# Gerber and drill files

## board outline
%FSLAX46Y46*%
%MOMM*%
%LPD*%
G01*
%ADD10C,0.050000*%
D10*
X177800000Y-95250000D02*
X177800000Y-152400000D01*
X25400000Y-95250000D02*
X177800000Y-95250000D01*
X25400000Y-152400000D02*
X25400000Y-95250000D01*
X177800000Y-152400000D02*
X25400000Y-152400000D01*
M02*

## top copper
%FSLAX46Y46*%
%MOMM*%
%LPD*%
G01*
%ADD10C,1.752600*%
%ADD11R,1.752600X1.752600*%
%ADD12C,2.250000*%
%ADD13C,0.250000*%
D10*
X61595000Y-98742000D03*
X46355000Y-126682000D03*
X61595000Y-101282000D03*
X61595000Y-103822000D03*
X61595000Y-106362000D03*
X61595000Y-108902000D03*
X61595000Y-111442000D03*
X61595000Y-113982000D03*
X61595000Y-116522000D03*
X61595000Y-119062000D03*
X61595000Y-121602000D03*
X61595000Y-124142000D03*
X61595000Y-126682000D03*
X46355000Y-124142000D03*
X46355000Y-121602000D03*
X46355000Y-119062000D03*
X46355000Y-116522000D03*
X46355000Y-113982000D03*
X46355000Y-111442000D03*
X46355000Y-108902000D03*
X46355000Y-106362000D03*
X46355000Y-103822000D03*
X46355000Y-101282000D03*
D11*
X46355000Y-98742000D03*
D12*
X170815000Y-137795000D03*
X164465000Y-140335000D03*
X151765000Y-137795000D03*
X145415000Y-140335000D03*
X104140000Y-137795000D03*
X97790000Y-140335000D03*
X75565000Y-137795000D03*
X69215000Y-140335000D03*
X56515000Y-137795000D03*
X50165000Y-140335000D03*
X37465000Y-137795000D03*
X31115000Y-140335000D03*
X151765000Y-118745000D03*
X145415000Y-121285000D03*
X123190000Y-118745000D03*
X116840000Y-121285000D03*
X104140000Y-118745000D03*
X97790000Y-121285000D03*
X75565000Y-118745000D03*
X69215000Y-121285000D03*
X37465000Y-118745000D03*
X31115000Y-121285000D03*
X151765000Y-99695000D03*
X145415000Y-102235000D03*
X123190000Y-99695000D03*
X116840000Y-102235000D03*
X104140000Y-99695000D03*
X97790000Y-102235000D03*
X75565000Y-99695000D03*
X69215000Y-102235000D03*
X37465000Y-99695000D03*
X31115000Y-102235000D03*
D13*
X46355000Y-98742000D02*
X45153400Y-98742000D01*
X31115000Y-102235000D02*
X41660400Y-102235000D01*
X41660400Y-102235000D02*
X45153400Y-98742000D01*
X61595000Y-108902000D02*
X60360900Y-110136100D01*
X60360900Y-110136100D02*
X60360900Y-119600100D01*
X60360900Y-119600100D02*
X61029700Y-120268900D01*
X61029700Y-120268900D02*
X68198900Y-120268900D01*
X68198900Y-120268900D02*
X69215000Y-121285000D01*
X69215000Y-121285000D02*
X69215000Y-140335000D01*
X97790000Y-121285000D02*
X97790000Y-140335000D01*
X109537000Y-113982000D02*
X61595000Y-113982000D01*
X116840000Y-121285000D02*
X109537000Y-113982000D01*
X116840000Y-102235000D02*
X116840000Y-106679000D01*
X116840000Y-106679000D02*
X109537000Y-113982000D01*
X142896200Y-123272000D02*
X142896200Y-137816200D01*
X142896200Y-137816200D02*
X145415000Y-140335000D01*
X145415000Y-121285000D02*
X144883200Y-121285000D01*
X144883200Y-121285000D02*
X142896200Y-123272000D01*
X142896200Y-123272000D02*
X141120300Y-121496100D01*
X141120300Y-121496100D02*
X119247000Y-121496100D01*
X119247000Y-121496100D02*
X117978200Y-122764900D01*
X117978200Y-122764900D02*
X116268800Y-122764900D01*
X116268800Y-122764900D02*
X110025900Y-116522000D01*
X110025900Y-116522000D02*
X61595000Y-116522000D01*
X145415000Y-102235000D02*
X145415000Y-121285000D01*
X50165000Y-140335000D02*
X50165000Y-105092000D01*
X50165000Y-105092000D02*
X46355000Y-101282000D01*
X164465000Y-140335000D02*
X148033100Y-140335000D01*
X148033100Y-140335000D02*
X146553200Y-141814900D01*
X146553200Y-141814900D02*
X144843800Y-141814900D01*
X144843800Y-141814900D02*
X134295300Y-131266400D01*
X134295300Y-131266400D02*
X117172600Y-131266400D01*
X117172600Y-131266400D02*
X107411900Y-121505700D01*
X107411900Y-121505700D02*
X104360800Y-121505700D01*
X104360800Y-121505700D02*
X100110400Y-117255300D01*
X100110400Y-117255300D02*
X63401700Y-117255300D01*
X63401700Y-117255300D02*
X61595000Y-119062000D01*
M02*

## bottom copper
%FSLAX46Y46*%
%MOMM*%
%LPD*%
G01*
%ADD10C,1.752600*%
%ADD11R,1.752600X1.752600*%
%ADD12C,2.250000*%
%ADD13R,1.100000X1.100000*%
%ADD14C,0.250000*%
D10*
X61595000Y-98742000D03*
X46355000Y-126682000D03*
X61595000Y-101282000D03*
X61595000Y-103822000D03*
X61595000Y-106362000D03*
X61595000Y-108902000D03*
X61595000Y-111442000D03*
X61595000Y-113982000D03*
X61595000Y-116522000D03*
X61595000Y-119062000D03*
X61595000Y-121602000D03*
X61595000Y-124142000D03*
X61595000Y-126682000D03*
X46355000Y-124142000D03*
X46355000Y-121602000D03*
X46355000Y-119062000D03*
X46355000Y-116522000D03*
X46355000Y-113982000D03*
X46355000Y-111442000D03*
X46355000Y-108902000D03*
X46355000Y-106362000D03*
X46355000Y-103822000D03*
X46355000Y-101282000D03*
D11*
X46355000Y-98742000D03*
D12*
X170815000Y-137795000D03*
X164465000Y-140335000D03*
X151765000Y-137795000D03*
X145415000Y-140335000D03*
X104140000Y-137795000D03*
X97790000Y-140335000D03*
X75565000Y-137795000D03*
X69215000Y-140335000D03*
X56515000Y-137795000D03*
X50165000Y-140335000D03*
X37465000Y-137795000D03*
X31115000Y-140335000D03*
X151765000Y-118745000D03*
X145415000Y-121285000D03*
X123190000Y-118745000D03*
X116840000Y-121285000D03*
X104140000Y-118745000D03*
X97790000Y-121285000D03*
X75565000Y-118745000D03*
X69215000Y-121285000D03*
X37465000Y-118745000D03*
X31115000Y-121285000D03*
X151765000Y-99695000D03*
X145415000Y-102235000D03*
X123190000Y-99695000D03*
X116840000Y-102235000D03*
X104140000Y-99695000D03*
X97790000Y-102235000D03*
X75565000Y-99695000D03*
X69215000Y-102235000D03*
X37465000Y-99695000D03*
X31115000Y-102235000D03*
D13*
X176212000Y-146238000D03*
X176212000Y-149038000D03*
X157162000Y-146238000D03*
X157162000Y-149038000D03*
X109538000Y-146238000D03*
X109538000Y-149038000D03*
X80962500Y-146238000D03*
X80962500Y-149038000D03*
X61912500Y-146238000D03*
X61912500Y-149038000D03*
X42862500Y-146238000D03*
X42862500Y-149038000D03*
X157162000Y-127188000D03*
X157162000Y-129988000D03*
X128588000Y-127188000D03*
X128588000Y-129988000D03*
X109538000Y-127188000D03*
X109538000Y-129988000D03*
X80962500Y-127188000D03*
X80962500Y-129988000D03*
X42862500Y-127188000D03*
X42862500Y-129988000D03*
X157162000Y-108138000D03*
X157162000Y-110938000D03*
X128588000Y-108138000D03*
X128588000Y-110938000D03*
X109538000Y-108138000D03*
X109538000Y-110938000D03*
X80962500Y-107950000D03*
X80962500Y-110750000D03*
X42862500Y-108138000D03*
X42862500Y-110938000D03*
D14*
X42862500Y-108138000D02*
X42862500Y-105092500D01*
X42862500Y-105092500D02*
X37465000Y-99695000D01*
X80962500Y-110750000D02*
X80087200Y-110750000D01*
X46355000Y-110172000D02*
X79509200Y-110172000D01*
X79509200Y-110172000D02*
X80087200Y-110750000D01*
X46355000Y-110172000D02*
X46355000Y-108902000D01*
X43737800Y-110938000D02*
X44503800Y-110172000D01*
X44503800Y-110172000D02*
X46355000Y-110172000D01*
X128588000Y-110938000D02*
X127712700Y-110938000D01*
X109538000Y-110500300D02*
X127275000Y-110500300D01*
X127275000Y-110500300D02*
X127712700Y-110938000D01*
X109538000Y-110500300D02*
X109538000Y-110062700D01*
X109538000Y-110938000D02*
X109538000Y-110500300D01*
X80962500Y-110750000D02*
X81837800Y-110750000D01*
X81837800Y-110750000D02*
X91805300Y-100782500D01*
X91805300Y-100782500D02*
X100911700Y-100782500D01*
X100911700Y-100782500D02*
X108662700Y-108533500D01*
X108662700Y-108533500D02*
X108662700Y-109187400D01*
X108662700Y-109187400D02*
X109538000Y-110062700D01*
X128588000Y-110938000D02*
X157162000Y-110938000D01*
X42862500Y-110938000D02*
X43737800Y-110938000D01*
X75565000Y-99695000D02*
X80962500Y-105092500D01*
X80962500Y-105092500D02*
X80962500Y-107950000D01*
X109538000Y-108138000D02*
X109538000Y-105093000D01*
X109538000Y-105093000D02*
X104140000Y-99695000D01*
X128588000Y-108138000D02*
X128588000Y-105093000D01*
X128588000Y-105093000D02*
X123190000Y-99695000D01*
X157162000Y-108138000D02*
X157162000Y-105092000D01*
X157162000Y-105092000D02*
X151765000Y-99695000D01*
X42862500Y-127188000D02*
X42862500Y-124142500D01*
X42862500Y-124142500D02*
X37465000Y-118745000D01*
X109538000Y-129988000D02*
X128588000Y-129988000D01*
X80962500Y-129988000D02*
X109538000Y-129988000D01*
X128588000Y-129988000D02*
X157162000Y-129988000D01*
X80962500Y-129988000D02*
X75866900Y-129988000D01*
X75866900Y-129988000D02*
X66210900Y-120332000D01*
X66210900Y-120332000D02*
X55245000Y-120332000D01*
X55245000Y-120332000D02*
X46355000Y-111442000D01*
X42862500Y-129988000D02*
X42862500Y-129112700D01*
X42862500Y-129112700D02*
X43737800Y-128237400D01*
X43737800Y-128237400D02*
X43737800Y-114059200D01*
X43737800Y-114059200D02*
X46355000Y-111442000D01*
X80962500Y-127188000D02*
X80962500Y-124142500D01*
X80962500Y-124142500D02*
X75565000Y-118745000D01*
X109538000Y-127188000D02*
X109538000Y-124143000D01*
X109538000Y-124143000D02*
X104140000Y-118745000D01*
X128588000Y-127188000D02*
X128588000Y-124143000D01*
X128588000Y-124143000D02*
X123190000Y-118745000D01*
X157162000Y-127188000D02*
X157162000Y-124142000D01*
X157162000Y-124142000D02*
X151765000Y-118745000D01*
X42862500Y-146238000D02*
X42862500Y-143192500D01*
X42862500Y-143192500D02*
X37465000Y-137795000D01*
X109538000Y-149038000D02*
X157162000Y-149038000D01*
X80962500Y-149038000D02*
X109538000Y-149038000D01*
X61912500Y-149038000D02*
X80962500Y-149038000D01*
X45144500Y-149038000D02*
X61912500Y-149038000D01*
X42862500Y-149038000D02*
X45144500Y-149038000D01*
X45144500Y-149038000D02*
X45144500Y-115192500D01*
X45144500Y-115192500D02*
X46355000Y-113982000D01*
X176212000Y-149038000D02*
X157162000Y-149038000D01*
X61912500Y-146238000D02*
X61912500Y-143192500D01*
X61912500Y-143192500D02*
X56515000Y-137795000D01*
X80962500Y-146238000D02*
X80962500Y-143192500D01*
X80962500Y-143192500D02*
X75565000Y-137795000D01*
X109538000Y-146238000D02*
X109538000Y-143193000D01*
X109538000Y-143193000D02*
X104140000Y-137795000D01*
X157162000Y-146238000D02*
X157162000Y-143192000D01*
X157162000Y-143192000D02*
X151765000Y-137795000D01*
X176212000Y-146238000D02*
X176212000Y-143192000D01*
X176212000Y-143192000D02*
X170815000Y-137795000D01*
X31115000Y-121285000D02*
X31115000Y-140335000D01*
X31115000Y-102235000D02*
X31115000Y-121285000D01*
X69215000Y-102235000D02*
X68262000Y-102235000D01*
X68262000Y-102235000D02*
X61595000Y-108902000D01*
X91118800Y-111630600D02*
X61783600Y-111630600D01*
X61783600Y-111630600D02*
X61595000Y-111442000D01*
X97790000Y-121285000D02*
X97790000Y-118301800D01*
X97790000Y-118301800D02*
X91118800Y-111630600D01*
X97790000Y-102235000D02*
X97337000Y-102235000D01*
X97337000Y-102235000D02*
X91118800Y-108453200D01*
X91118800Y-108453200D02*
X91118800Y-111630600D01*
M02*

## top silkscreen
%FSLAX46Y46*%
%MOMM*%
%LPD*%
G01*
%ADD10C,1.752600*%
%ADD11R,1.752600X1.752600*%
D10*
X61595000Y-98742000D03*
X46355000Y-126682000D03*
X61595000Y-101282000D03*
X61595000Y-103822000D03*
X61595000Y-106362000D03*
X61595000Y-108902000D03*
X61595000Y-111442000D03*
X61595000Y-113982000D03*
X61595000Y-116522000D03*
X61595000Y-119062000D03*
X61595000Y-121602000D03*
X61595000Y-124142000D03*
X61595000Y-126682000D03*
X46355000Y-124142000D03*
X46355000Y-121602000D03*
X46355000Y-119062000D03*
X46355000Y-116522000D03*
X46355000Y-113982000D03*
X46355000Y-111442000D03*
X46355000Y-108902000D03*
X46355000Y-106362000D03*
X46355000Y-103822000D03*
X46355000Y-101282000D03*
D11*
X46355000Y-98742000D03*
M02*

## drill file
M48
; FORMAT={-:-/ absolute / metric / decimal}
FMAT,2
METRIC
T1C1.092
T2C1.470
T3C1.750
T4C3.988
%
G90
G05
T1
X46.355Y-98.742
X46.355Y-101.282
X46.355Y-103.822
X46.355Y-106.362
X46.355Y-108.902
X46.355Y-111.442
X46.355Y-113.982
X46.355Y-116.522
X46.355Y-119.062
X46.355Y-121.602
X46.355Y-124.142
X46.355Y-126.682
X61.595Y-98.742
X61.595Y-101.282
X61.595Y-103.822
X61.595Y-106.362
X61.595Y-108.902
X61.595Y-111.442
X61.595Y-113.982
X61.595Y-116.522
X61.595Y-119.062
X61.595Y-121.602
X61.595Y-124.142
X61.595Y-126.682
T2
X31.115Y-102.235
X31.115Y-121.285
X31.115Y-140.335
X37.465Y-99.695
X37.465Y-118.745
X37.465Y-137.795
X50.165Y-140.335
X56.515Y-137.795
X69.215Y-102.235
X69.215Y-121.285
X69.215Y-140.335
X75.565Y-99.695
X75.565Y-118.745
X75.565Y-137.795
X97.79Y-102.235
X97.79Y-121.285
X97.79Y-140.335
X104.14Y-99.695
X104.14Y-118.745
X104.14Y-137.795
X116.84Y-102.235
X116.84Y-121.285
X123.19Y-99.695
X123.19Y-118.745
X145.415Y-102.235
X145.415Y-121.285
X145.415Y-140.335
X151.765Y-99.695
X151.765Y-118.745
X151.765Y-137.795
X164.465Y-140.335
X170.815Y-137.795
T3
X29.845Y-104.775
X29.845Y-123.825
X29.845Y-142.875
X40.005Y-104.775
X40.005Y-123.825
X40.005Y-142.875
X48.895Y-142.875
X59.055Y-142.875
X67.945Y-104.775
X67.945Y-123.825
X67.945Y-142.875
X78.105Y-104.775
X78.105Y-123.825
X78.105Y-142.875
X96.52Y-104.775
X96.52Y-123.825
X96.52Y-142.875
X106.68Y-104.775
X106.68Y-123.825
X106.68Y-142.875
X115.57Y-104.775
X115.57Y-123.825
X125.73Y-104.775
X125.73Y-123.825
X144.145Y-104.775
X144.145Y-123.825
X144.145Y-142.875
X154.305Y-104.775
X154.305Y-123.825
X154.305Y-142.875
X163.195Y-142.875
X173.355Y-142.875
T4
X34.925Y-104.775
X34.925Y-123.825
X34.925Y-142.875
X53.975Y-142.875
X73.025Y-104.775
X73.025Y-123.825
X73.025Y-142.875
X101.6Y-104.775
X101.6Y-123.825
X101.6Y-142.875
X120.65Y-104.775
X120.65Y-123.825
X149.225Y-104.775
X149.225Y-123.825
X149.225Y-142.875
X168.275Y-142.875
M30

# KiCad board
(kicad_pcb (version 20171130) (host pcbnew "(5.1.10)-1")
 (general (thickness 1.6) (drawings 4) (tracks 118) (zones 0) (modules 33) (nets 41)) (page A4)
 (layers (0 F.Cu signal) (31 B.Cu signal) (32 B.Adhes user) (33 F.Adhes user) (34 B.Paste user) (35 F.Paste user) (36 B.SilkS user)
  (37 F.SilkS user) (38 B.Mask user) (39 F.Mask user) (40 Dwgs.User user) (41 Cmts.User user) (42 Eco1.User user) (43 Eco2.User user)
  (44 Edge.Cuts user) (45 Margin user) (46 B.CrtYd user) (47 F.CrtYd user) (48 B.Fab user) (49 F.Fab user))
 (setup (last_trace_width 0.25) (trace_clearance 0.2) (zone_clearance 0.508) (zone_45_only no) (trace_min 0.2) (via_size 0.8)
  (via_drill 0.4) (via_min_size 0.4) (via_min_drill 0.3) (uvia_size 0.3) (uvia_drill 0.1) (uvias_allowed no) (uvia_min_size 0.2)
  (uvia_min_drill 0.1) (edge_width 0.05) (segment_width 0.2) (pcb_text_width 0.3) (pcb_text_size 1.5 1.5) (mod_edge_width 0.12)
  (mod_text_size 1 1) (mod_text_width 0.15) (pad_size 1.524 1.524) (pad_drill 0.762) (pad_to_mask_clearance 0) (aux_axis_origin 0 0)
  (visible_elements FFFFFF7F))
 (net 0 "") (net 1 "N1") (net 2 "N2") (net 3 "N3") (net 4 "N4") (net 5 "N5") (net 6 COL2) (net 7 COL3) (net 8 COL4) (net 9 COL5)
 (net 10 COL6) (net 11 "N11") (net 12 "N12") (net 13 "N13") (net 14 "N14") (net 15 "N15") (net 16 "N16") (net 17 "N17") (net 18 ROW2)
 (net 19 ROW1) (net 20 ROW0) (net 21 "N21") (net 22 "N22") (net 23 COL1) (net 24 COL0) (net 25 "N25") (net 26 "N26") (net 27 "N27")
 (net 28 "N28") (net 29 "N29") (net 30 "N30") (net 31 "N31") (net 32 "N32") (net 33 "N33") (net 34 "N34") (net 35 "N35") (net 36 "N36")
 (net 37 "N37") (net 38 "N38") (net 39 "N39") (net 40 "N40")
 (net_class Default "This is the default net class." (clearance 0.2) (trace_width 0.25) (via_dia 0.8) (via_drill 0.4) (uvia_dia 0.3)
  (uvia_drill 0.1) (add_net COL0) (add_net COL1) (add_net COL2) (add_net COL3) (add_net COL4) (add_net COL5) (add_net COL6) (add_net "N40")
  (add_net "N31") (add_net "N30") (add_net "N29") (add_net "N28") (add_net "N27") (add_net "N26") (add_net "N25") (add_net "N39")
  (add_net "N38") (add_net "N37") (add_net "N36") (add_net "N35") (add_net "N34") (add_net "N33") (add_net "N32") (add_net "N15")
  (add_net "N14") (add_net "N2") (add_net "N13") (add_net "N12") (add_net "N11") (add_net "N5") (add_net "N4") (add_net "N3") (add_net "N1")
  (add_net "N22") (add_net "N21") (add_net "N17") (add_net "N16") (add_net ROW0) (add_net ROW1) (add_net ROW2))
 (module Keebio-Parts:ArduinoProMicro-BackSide (layer F.Cu) (at 53.975 112.712 270)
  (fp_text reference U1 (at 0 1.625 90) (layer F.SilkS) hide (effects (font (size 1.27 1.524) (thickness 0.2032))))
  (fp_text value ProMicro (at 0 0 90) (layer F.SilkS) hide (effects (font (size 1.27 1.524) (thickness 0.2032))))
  (pad 24 thru_hole circle (at -13.97 -7.62 270) (size 1.7526 1.7526) (drill 1.0922) (layers *.Cu *.SilkS *.Mask) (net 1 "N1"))
  (pad 12 thru_hole circle (at 13.97 7.62 270) (size 1.7526 1.7526) (drill 1.0922) (layers *.Cu *.SilkS *.Mask) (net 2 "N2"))
  (pad 23 thru_hole circle (at -11.43 -7.62 270) (size 1.7526 1.7526) (drill 1.0922) (layers *.Cu *.SilkS *.Mask) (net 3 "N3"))
  (pad 22 thru_hole circle (at -8.89 -7.62 270) (size 1.7526 1.7526) (drill 1.0922) (layers *.Cu *.SilkS *.Mask) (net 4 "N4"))
  (pad 21 thru_hole circle (at -6.35 -7.62 270) (size 1.7526 1.7526) (drill 1.0922) (layers *.Cu *.SilkS *.Mask) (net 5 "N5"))
  (pad 20 thru_hole circle (at -3.81 -7.62 270) (size 1.7526 1.7526) (drill 1.0922) (layers *.Cu *.SilkS *.Mask) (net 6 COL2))
  (pad 19 thru_hole circle (at -1.27 -7.62 270) (size 1.7526 1.7526) (drill 1.0922) (layers *.Cu *.SilkS *.Mask) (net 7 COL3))
  (pad 18 thru_hole circle (at 1.27 -7.62 270) (size 1.7526 1.7526) (drill 1.0922) (layers *.Cu *.SilkS *.Mask) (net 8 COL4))
  (pad 17 thru_hole circle (at 3.81 -7.62 270) (size 1.7526 1.7526) (drill 1.0922) (layers *.Cu *.SilkS *.Mask) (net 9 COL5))
  (pad 16 thru_hole circle (at 6.35 -7.62 270) (size 1.7526 1.7526) (drill 1.0922) (layers *.Cu *.SilkS *.Mask) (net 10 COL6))
  (pad 15 thru_hole circle (at 8.89 -7.62 270) (size 1.7526 1.7526) (drill 1.0922) (layers *.Cu *.SilkS *.Mask) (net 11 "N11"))
  (pad 14 thru_hole circle (at 11.43 -7.62 270) (size 1.7526 1.7526) (drill 1.0922) (layers *.Cu *.SilkS *.Mask) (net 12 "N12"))
  (pad 13 thru_hole circle (at 13.97 -7.62 270) (size 1.7526 1.7526) (drill 1.0922) (layers *.Cu *.SilkS *.Mask) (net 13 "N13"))
  (pad 11 thru_hole circle (at 11.43 7.62 270) (size 1.7526 1.7526) (drill 1.0922) (layers *.Cu *.SilkS *.Mask) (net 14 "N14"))
  (pad 10 thru_hole circle (at 8.89 7.62 270) (size 1.7526 1.7526) (drill 1.0922) (layers *.Cu *.SilkS *.Mask) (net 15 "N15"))
  (pad 9 thru_hole circle (at 6.35 7.62 270) (size 1.7526 1.7526) (drill 1.0922) (layers *.Cu *.SilkS *.Mask) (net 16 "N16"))
  (pad 8 thru_hole circle (at 3.81 7.62 270) (size 1.7526 1.7526) (drill 1.0922) (layers *.Cu *.SilkS *.Mask) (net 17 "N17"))
  (pad 7 thru_hole circle (at 1.27 7.62 270) (size 1.7526 1.7526) (drill 1.0922) (layers *.Cu *.SilkS *.Mask) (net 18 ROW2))
  (pad 6 thru_hole circle (at -1.27 7.62 270) (size 1.7526 1.7526) (drill 1.0922) (layers *.Cu *.SilkS *.Mask) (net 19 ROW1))
  (pad 5 thru_hole circle (at -3.81 7.62 270) (size 1.7526 1.7526) (drill 1.0922) (layers *.Cu *.SilkS *.Mask) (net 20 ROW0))
  (pad 4 thru_hole circle (at -6.35 7.62 270) (size 1.7526 1.7526) (drill 1.0922) (layers *.Cu *.SilkS *.Mask) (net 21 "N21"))
  (pad 3 thru_hole circle (at -8.89 7.62 270) (size 1.7526 1.7526) (drill 1.0922) (layers *.Cu *.SilkS *.Mask) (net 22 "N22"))
  (pad 2 thru_hole circle (at -11.43 7.62 270) (size 1.7526 1.7526) (drill 1.0922) (layers *.Cu *.SilkS *.Mask) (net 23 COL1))
  (pad 1 thru_hole rect (at -13.97 7.62 270) (size 1.7526 1.7526) (drill 1.0922) (layers *.Cu *.SilkS *.Mask) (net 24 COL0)))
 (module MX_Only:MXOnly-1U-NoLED (layer F.Cu) (at 168.275 142.875)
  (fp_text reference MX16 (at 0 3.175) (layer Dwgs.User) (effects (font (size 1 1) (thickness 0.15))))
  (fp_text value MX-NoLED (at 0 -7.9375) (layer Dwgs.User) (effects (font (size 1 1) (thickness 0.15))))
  (pad 2 thru_hole circle (at 2.54 -5.08) (size 2.25 2.25) (drill 1.47) (layers *.Cu B.Mask) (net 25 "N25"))
  (pad "" np_thru_hole circle (at 0 0) (size 3.9878 3.9878) (drill 3.9878) (layers *.Cu *.Mask))
  (pad 1 thru_hole circle (at -3.81 -2.54) (size 2.25 2.25) (drill 1.47) (layers *.Cu B.Mask) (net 10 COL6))
  (pad "" np_thru_hole circle (at -5.08 0 48.0996) (size 1.75 1.75) (drill 1.75) (layers *.Cu *.Mask))
  (pad "" np_thru_hole circle (at 5.08 0 48.0996) (size 1.75 1.75) (drill 1.75) (layers *.Cu *.Mask)))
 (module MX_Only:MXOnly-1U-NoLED (layer F.Cu) (at 149.225 142.875)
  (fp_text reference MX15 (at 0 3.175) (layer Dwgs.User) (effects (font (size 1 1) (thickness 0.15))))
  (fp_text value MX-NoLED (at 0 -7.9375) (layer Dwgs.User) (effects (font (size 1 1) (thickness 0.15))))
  (pad 2 thru_hole circle (at 2.54 -5.08) (size 2.25 2.25) (drill 1.47) (layers *.Cu B.Mask) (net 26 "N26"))
  (pad "" np_thru_hole circle (at 0 0) (size 3.9878 3.9878) (drill 3.9878) (layers *.Cu *.Mask))
  (pad 1 thru_hole circle (at -3.81 -2.54) (size 2.25 2.25) (drill 1.47) (layers *.Cu B.Mask) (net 9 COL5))
  (pad "" np_thru_hole circle (at -5.08 0 48.0996) (size 1.75 1.75) (drill 1.75) (layers *.Cu *.Mask))
  (pad "" np_thru_hole circle (at 5.08 0 48.0996) (size 1.75 1.75) (drill 1.75) (layers *.Cu *.Mask)))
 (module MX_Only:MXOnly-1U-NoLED (layer F.Cu) (at 101.6 142.875)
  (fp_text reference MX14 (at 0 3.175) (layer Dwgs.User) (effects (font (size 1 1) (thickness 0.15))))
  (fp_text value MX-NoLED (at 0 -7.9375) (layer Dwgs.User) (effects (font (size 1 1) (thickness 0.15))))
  (pad 2 thru_hole circle (at 2.54 -5.08) (size 2.25 2.25) (drill 1.47) (layers *.Cu B.Mask) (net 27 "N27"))
  (pad "" np_thru_hole circle (at 0 0) (size 3.9878 3.9878) (drill 3.9878) (layers *.Cu *.Mask))
  (pad 1 thru_hole circle (at -3.81 -2.54) (size 2.25 2.25) (drill 1.47) (layers *.Cu B.Mask) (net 7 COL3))
  (pad "" np_thru_hole circle (at -5.08 0 48.0996) (size 1.75 1.75) (drill 1.75) (layers *.Cu *.Mask))
  (pad "" np_thru_hole circle (at 5.08 0 48.0996) (size 1.75 1.75) (drill 1.75) (layers *.Cu *.Mask)))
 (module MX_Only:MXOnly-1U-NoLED (layer F.Cu) (at 73.025 142.875)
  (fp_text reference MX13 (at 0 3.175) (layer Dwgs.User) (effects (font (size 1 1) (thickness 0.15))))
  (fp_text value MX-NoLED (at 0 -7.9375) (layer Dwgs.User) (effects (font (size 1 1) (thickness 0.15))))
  (pad 2 thru_hole circle (at 2.54 -5.08) (size 2.25 2.25) (drill 1.47) (layers *.Cu B.Mask) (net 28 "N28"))
  (pad "" np_thru_hole circle (at 0 0) (size 3.9878 3.9878) (drill 3.9878) (layers *.Cu *.Mask))
  (pad 1 thru_hole circle (at -3.81 -2.54) (size 2.25 2.25) (drill 1.47) (layers *.Cu B.Mask) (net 6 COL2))
  (pad "" np_thru_hole circle (at -5.08 0 48.0996) (size 1.75 1.75) (drill 1.75) (layers *.Cu *.Mask))
  (pad "" np_thru_hole circle (at 5.08 0 48.0996) (size 1.75 1.75) (drill 1.75) (layers *.Cu *.Mask)))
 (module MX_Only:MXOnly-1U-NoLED (layer F.Cu) (at 53.975 142.875)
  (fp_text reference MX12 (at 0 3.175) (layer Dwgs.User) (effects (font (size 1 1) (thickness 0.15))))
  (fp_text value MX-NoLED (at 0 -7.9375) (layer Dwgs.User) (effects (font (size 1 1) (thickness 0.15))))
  (pad 2 thru_hole circle (at 2.54 -5.08) (size 2.25 2.25) (drill 1.47) (layers *.Cu B.Mask) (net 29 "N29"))
  (pad "" np_thru_hole circle (at 0 0) (size 3.9878 3.9878) (drill 3.9878) (layers *.Cu *.Mask))
  (pad 1 thru_hole circle (at -3.81 -2.54) (size 2.25 2.25) (drill 1.47) (layers *.Cu B.Mask) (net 23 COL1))
  (pad "" np_thru_hole circle (at -5.08 0 48.0996) (size 1.75 1.75) (drill 1.75) (layers *.Cu *.Mask))
  (pad "" np_thru_hole circle (at 5.08 0 48.0996) (size 1.75 1.75) (drill 1.75) (layers *.Cu *.Mask)))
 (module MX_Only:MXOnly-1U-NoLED (layer F.Cu) (at 34.925 142.875)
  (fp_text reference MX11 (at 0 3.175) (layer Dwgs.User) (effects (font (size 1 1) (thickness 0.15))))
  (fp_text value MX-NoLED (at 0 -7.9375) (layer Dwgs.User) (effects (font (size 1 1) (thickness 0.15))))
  (pad 2 thru_hole circle (at 2.54 -5.08) (size 2.25 2.25) (drill 1.47) (layers *.Cu B.Mask) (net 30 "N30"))
  (pad "" np_thru_hole circle (at 0 0) (size 3.9878 3.9878) (drill 3.9878) (layers *.Cu *.Mask))
  (pad 1 thru_hole circle (at -3.81 -2.54) (size 2.25 2.25) (drill 1.47) (layers *.Cu B.Mask) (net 24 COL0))
  (pad "" np_thru_hole circle (at -5.08 0 48.0996) (size 1.75 1.75) (drill 1.75) (layers *.Cu *.Mask))
  (pad "" np_thru_hole circle (at 5.08 0 48.0996) (size 1.75 1.75) (drill 1.75) (layers *.Cu *.Mask)))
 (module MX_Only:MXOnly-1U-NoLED (layer F.Cu) (at 149.225 123.825)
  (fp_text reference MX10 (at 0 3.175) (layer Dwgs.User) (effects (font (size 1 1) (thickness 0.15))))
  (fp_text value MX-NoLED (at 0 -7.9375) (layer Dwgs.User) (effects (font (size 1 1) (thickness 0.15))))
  (pad 2 thru_hole circle (at 2.54 -5.08) (size 2.25 2.25) (drill 1.47) (layers *.Cu B.Mask) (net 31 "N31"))
  (pad "" np_thru_hole circle (at 0 0) (size 3.9878 3.9878) (drill 3.9878) (layers *.Cu *.Mask))
  (pad 1 thru_hole circle (at -3.81 -2.54) (size 2.25 2.25) (drill 1.47) (layers *.Cu B.Mask) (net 9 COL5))
  (pad "" np_thru_hole circle (at -5.08 0 48.0996) (size 1.75 1.75) (drill 1.75) (layers *.Cu *.Mask))
  (pad "" np_thru_hole circle (at 5.08 0 48.0996) (size 1.75 1.75) (drill 1.75) (layers *.Cu *.Mask)))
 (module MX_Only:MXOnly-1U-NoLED (layer F.Cu) (at 120.65 123.825)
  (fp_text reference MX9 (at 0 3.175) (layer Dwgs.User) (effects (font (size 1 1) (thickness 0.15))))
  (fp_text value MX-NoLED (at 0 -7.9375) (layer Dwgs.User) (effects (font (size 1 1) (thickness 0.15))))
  (pad 2 thru_hole circle (at 2.54 -5.08) (size 2.25 2.25) (drill 1.47) (layers *.Cu B.Mask) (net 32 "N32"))
  (pad "" np_thru_hole circle (at 0 0) (size 3.9878 3.9878) (drill 3.9878) (layers *.Cu *.Mask))
  (pad 1 thru_hole circle (at -3.81 -2.54) (size 2.25 2.25) (drill 1.47) (layers *.Cu B.Mask) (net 8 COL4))
  (pad "" np_thru_hole circle (at -5.08 0 48.0996) (size 1.75 1.75) (drill 1.75) (layers *.Cu *.Mask))
  (pad "" np_thru_hole circle (at 5.08 0 48.0996) (size 1.75 1.75) (drill 1.75) (layers *.Cu *.Mask)))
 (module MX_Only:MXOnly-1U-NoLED (layer F.Cu) (at 101.6 123.825)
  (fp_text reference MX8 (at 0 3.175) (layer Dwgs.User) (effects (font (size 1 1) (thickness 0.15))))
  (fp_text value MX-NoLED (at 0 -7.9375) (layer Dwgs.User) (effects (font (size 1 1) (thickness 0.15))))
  (pad 2 thru_hole circle (at 2.54 -5.08) (size 2.25 2.25) (drill 1.47) (layers *.Cu B.Mask) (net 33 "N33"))
  (pad "" np_thru_hole circle (at 0 0) (size 3.9878 3.9878) (drill 3.9878) (layers *.Cu *.Mask))
  (pad 1 thru_hole circle (at -3.81 -2.54) (size 2.25 2.25) (drill 1.47) (layers *.Cu B.Mask) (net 7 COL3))
  (pad "" np_thru_hole circle (at -5.08 0 48.0996) (size 1.75 1.75) (drill 1.75) (layers *.Cu *.Mask))
  (pad "" np_thru_hole circle (at 5.08 0 48.0996) (size 1.75 1.75) (drill 1.75) (layers *.Cu *.Mask)))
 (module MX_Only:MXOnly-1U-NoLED (layer F.Cu) (at 73.025 123.825)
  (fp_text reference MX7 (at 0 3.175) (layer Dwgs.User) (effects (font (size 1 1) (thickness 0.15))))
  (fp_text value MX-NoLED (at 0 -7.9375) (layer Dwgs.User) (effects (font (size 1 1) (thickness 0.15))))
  (pad 2 thru_hole circle (at 2.54 -5.08) (size 2.25 2.25) (drill 1.47) (layers *.Cu B.Mask) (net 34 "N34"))
  (pad "" np_thru_hole circle (at 0 0) (size 3.9878 3.9878) (drill 3.9878) (layers *.Cu *.Mask))
  (pad 1 thru_hole circle (at -3.81 -2.54) (size 2.25 2.25) (drill 1.47) (layers *.Cu B.Mask) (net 6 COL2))
  (pad "" np_thru_hole circle (at -5.08 0 48.0996) (size 1.75 1.75) (drill 1.75) (layers *.Cu *.Mask))
  (pad "" np_thru_hole circle (at 5.08 0 48.0996) (size 1.75 1.75) (drill 1.75) (layers *.Cu *.Mask)))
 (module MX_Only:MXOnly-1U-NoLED (layer F.Cu) (at 34.925 123.825)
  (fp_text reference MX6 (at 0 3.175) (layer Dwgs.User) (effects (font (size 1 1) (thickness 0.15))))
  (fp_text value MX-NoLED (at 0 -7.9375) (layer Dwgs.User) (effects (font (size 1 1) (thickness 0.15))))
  (pad 2 thru_hole circle (at 2.54 -5.08) (size 2.25 2.25) (drill 1.47) (layers *.Cu B.Mask) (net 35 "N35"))
  (pad "" np_thru_hole circle (at 0 0) (size 3.9878 3.9878) (drill 3.9878) (layers *.Cu *.Mask))
  (pad 1 thru_hole circle (at -3.81 -2.54) (size 2.25 2.25) (drill 1.47) (layers *.Cu B.Mask) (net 24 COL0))
  (pad "" np_thru_hole circle (at -5.08 0 48.0996) (size 1.75 1.75) (drill 1.75) (layers *.Cu *.Mask))
  (pad "" np_thru_hole circle (at 5.08 0 48.0996) (size 1.75 1.75) (drill 1.75) (layers *.Cu *.Mask)))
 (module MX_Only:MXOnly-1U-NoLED (layer F.Cu) (at 149.225 104.775)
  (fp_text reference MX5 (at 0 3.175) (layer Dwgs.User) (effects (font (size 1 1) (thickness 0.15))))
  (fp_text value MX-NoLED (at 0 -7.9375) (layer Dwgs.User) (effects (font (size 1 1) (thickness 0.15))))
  (pad 2 thru_hole circle (at 2.54 -5.08) (size 2.25 2.25) (drill 1.47) (layers *.Cu B.Mask) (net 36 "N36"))
  (pad "" np_thru_hole circle (at 0 0) (size 3.9878 3.9878) (drill 3.9878) (layers *.Cu *.Mask))
  (pad 1 thru_hole circle (at -3.81 -2.54) (size 2.25 2.25) (drill 1.47) (layers *.Cu B.Mask) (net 9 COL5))
  (pad "" np_thru_hole circle (at -5.08 0 48.0996) (size 1.75 1.75) (drill 1.75) (layers *.Cu *.Mask))
  (pad "" np_thru_hole circle (at 5.08 0 48.0996) (size 1.75 1.75) (drill 1.75) (layers *.Cu *.Mask)))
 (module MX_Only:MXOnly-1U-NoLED (layer F.Cu) (at 120.65 104.775)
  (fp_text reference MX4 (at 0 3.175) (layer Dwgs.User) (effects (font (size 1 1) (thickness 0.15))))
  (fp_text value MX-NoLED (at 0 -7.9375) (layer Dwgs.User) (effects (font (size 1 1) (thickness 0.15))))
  (pad 2 thru_hole circle (at 2.54 -5.08) (size 2.25 2.25) (drill 1.47) (layers *.Cu B.Mask) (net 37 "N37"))
  (pad "" np_thru_hole circle (at 0 0) (size 3.9878 3.9878) (drill 3.9878) (layers *.Cu *.Mask))
  (pad 1 thru_hole circle (at -3.81 -2.54) (size 2.25 2.25) (drill 1.47) (layers *.Cu B.Mask) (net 8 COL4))
  (pad "" np_thru_hole circle (at -5.08 0 48.0996) (size 1.75 1.75) (drill 1.75) (layers *.Cu *.Mask))
  (pad "" np_thru_hole circle (at 5.08 0 48.0996) (size 1.75 1.75) (drill 1.75) (layers *.Cu *.Mask)))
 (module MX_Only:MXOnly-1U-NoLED (layer F.Cu) (at 101.6 104.775)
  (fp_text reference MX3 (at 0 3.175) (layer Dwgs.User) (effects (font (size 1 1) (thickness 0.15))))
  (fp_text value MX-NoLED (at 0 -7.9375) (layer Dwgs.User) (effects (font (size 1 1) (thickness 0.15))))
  (pad 2 thru_hole circle (at 2.54 -5.08) (size 2.25 2.25) (drill 1.47) (layers *.Cu B.Mask) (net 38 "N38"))
  (pad "" np_thru_hole circle (at 0 0) (size 3.9878 3.9878) (drill 3.9878) (layers *.Cu *.Mask))
  (pad 1 thru_hole circle (at -3.81 -2.54) (size 2.25 2.25) (drill 1.47) (layers *.Cu B.Mask) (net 7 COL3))
  (pad "" np_thru_hole circle (at -5.08 0 48.0996) (size 1.75 1.75) (drill 1.75) (layers *.Cu *.Mask))
  (pad "" np_thru_hole circle (at 5.08 0 48.0996) (size 1.75 1.75) (drill 1.75) (layers *.Cu *.Mask)))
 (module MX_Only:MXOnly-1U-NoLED (layer F.Cu) (at 73.025 104.775)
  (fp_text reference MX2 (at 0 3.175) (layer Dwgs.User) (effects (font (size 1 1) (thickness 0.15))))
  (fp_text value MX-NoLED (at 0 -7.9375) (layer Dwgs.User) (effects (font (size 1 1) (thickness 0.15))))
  (pad 2 thru_hole circle (at 2.54 -5.08) (size 2.25 2.25) (drill 1.47) (layers *.Cu B.Mask) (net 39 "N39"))
  (pad "" np_thru_hole circle (at 0 0) (size 3.9878 3.9878) (drill 3.9878) (layers *.Cu *.Mask))
  (pad 1 thru_hole circle (at -3.81 -2.54) (size 2.25 2.25) (drill 1.47) (layers *.Cu B.Mask) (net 6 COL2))
  (pad "" np_thru_hole circle (at -5.08 0 48.0996) (size 1.75 1.75) (drill 1.75) (layers *.Cu *.Mask))
  (pad "" np_thru_hole circle (at 5.08 0 48.0996) (size 1.75 1.75) (drill 1.75) (layers *.Cu *.Mask)))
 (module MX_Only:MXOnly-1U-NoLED (layer F.Cu) (at 34.925 104.775)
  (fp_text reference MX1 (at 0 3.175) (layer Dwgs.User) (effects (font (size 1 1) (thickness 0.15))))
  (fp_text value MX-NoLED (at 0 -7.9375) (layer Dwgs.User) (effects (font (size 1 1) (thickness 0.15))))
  (pad 2 thru_hole circle (at 2.54 -5.08) (size 2.25 2.25) (drill 1.47) (layers *.Cu B.Mask) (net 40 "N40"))
  (pad "" np_thru_hole circle (at 0 0) (size 3.9878 3.9878) (drill 3.9878) (layers *.Cu *.Mask))
  (pad 1 thru_hole circle (at -3.81 -2.54) (size 2.25 2.25) (drill 1.47) (layers *.Cu B.Mask) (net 24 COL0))
  (pad "" np_thru_hole circle (at -5.08 0 48.0996) (size 1.75 1.75) (drill 1.75) (layers *.Cu *.Mask))
  (pad "" np_thru_hole circle (at 5.08 0 48.0996) (size 1.75 1.75) (drill 1.75) (layers *.Cu *.Mask)))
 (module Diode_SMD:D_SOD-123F (layer B.Cu) (at 176.212 147.638 90)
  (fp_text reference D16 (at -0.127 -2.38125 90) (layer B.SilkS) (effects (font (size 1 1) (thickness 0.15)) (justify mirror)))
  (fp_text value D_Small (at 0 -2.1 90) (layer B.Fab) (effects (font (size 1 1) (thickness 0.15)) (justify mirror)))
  (pad 2 smd rect (at 1.4 0 90) (size 1.1 1.1) (layers B.Cu B.Paste B.Mask) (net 25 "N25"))
  (pad 1 smd rect (at -1.4 0 90) (size 1.1 1.1) (layers B.Cu B.Paste B.Mask) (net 18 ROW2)))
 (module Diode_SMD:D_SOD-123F (layer B.Cu) (at 157.162 147.638 90)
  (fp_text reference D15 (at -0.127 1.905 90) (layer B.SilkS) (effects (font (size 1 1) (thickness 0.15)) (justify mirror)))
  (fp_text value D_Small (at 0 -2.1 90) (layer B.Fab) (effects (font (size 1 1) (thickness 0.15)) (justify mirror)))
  (pad 2 smd rect (at 1.4 0 90) (size 1.1 1.1) (layers B.Cu B.Paste B.Mask) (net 26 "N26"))
  (pad 1 smd rect (at -1.4 0 90) (size 1.1 1.1) (layers B.Cu B.Paste B.Mask) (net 18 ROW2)))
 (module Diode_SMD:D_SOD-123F (layer B.Cu) (at 109.538 147.638 90)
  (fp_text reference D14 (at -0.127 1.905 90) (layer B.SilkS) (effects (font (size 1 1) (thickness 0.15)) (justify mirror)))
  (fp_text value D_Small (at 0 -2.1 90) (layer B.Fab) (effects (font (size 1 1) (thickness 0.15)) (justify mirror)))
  (pad 2 smd rect (at 1.4 0 90) (size 1.1 1.1) (layers B.Cu B.Paste B.Mask) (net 27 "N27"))
  (pad 1 smd rect (at -1.4 0 90) (size 1.1 1.1) (layers B.Cu B.Paste B.Mask) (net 18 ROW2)))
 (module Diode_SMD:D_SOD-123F (layer B.Cu) (at 80.9625 147.638 90)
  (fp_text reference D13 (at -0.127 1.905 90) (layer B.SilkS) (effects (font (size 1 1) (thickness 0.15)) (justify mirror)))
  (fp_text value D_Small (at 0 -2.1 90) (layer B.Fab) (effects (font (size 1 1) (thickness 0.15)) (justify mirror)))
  (pad 2 smd rect (at 1.4 0 90) (size 1.1 1.1) (layers B.Cu B.Paste B.Mask) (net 28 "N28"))
  (pad 1 smd rect (at -1.4 0 90) (size 1.1 1.1) (layers B.Cu B.Paste B.Mask) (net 18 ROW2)))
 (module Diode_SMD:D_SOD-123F (layer B.Cu) (at 61.9125 147.638 90)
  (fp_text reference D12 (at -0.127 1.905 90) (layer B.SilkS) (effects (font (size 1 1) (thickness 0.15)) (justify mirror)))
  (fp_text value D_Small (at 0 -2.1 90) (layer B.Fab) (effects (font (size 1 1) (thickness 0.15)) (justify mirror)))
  (pad 2 smd rect (at 1.4 0 90) (size 1.1 1.1) (layers B.Cu B.Paste B.Mask) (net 29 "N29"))
  (pad 1 smd rect (at -1.4 0 90) (size 1.1 1.1) (layers B.Cu B.Paste B.Mask) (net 18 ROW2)))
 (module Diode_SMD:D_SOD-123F (layer B.Cu) (at 42.8625 147.638 90)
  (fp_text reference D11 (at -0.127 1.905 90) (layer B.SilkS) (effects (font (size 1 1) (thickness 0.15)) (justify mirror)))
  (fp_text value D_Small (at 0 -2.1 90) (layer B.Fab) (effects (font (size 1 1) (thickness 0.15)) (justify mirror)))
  (pad 2 smd rect (at 1.4 0 90) (size 1.1 1.1) (layers B.Cu B.Paste B.Mask) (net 30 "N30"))
  (pad 1 smd rect (at -1.4 0 90) (size 1.1 1.1) (layers B.Cu B.Paste B.Mask) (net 18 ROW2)))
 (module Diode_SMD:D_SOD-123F (layer B.Cu) (at 157.162 128.588 90)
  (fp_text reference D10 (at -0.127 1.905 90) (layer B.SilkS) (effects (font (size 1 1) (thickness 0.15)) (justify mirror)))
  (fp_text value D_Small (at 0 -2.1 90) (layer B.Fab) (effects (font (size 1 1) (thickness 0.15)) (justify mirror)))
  (pad 2 smd rect (at 1.4 0 90) (size 1.1 1.1) (layers B.Cu B.Paste B.Mask) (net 31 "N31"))
  (pad 1 smd rect (at -1.4 0 90) (size 1.1 1.1) (layers B.Cu B.Paste B.Mask) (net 19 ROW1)))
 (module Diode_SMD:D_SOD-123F (layer B.Cu) (at 128.588 128.588 90)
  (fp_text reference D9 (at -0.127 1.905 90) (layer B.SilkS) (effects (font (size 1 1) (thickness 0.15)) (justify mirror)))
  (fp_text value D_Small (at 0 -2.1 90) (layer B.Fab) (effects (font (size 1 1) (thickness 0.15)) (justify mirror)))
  (pad 2 smd rect (at 1.4 0 90) (size 1.1 1.1) (layers B.Cu B.Paste B.Mask) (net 32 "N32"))
  (pad 1 smd rect (at -1.4 0 90) (size 1.1 1.1) (layers B.Cu B.Paste B.Mask) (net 19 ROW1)))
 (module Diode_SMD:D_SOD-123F (layer B.Cu) (at 109.538 128.588 90)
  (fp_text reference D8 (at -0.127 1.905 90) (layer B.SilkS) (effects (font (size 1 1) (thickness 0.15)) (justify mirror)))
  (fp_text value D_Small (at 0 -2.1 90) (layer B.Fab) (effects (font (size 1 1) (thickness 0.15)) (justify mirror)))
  (pad 2 smd rect (at 1.4 0 90) (size 1.1 1.1) (layers B.Cu B.Paste B.Mask) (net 33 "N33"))
  (pad 1 smd rect (at -1.4 0 90) (size 1.1 1.1) (layers B.Cu B.Paste B.Mask) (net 19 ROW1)))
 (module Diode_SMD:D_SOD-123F (layer B.Cu) (at 80.9625 128.588 90)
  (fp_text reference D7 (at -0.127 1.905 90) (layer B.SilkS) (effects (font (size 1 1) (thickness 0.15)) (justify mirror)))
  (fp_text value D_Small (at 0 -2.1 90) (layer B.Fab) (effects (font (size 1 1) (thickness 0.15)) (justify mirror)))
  (pad 2 smd rect (at 1.4 0 90) (size 1.1 1.1) (layers B.Cu B.Paste B.Mask) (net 34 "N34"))
  (pad 1 smd rect (at -1.4 0 90) (size 1.1 1.1) (layers B.Cu B.Paste B.Mask) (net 19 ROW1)))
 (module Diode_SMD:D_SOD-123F (layer B.Cu) (at 42.8625 128.588 90)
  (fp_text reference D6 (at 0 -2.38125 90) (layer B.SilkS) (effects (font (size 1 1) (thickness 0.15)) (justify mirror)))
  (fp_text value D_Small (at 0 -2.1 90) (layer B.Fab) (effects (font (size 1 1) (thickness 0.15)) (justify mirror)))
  (pad 2 smd rect (at 1.4 0 90) (size 1.1 1.1) (layers B.Cu B.Paste B.Mask) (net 35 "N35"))
  (pad 1 smd rect (at -1.4 0 90) (size 1.1 1.1) (layers B.Cu B.Paste B.Mask) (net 19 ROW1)))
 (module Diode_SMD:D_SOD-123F (layer B.Cu) (at 157.162 109.538 90)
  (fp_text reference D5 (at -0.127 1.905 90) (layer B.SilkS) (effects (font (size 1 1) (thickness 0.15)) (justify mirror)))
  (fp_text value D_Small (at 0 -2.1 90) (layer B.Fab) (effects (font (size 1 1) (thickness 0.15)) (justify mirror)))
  (pad 2 smd rect (at 1.4 0 90) (size 1.1 1.1) (layers B.Cu B.Paste B.Mask) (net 36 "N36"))
  (pad 1 smd rect (at -1.4 0 90) (size 1.1 1.1) (layers B.Cu B.Paste B.Mask) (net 20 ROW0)))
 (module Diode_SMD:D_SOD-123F (layer B.Cu) (at 128.588 109.538 90)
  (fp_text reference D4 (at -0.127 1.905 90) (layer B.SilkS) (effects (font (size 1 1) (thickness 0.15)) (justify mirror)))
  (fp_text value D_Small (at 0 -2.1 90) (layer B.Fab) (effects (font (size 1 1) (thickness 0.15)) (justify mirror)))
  (pad 2 smd rect (at 1.4 0 90) (size 1.1 1.1) (layers B.Cu B.Paste B.Mask) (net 37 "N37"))
  (pad 1 smd rect (at -1.4 0 90) (size 1.1 1.1) (layers B.Cu B.Paste B.Mask) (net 20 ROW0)))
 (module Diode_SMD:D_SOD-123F (layer B.Cu) (at 109.538 109.538 90)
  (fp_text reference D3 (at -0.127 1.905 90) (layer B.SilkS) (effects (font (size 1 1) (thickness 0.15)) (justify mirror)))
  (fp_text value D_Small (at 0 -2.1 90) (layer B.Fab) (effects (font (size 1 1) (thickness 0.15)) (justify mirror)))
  (pad 2 smd rect (at 1.4 0 90) (size 1.1 1.1) (layers B.Cu B.Paste B.Mask) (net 38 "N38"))
  (pad 1 smd rect (at -1.4 0 90) (size 1.1 1.1) (layers B.Cu B.Paste B.Mask) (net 20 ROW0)))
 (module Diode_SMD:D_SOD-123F (layer B.Cu) (at 80.9625 109.35 90)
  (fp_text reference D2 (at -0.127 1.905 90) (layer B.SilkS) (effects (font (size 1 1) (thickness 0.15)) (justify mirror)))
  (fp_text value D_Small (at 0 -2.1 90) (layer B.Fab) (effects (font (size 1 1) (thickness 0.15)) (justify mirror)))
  (pad 2 smd rect (at 1.4 0 90) (size 1.1 1.1) (layers B.Cu B.Paste B.Mask) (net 39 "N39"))
  (pad 1 smd rect (at -1.4 0 90) (size 1.1 1.1) (layers B.Cu B.Paste B.Mask) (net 20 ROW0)))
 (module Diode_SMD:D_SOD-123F (layer B.Cu) (at 42.8625 109.538 90)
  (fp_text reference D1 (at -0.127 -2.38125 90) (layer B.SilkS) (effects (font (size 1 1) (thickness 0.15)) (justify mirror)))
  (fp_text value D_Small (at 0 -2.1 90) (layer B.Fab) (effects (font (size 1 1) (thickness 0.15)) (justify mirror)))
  (pad 2 smd rect (at 1.4 0 90) (size 1.1 1.1) (layers B.Cu B.Paste B.Mask) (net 40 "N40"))
  (pad 1 smd rect (at -1.4 0 90) (size 1.1 1.1) (layers B.Cu B.Paste B.Mask) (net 20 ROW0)))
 (gr_line (start 177.8 95.25) (end 177.8 152.4) (layer Edge.Cuts) (width 0.05))
 (gr_line (start 25.4 95.25) (end 177.8 95.25) (layer Edge.Cuts) (width 0.05))
 (gr_line (start 25.4 152.4) (end 25.4 95.25) (layer Edge.Cuts) (width 0.05))
 (gr_line (start 177.8 152.4) (end 25.4 152.4) (layer Edge.Cuts) (width 0.05))
 (segment (start 42.8625 108.138) (end 42.8625 105.0925) (width 0.25) (layer B.Cu) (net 40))
 (segment (start 42.8625 105.0925) (end 37.465 99.695) (width 0.25) (layer B.Cu) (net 40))
 (segment (start 80.9625 110.75) (end 80.0872 110.75) (width 0.25) (layer B.Cu) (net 20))
 (segment (start 46.355 110.172) (end 79.5092 110.172) (width 0.25) (layer B.Cu) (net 20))
 (segment (start 79.5092 110.172) (end 80.0872 110.75) (width 0.25) (layer B.Cu) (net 20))
 (segment (start 46.355 110.172) (end 46.355 108.902) (width 0.25) (layer B.Cu) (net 20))
 (segment (start 43.7378 110.938) (end 44.5038 110.172) (width 0.25) (layer B.Cu) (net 20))
 (segment (start 44.5038 110.172) (end 46.355 110.172) (width 0.25) (layer B.Cu) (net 20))
 (segment (start 128.588 110.938) (end 127.7127 110.938) (width 0.25) (layer B.Cu) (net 20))
 (segment (start 109.538 110.5003) (end 127.275 110.5003) (width 0.25) (layer B.Cu) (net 20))
 (segment (start 127.275 110.5003) (end 127.7127 110.938) (width 0.25) (layer B.Cu) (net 20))
 (segment (start 109.538 110.5003) (end 109.538 110.0627) (width 0.25) (layer B.Cu) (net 20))
 (segment (start 109.538 110.938) (end 109.538 110.5003) (width 0.25) (layer B.Cu) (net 20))
 (segment (start 80.9625 110.75) (end 81.8378 110.75) (width 0.25) (layer B.Cu) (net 20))
 (segment (start 81.8378 110.75) (end 91.8053 100.7825) (width 0.25) (layer B.Cu) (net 20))
 (segment (start 91.8053 100.7825) (end 100.9117 100.7825) (width 0.25) (layer B.Cu) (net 20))
 (segment (start 100.9117 100.7825) (end 108.6627 108.5335) (width 0.25) (layer B.Cu) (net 20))
 (segment (start 108.6627 108.5335) (end 108.6627 109.1874) (width 0.25) (layer B.Cu) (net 20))
 (segment (start 108.6627 109.1874) (end 109.538 110.0627) (width 0.25) (layer B.Cu) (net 20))
 (segment (start 128.588 110.938) (end 157.162 110.938) (width 0.25) (layer B.Cu) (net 20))
 (segment (start 42.8625 110.938) (end 43.7378 110.938) (width 0.25) (layer B.Cu) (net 20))
 (segment (start 75.565 99.695) (end 80.9625 105.0925) (width 0.25) (layer B.Cu) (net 39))
 (segment (start 80.9625 105.0925) (end 80.9625 107.95) (width 0.25) (layer B.Cu) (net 39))
 (segment (start 109.538 108.138) (end 109.538 105.093) (width 0.25) (layer B.Cu) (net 38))
 (segment (start 109.538 105.093) (end 104.14 99.695) (width 0.25) (layer B.Cu) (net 38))
 (segment (start 128.588 108.138) (end 128.588 105.093) (width 0.25) (layer B.Cu) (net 37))
 (segment (start 128.588 105.093) (end 123.19 99.695) (width 0.25) (layer B.Cu) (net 37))
 (segment (start 157.162 108.138) (end 157.162 105.092) (width 0.25) (layer B.Cu) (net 36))
 (segment (start 157.162 105.092) (end 151.765 99.695) (width 0.25) (layer B.Cu) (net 36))
 (segment (start 42.8625 127.188) (end 42.8625 124.1425) (width 0.25) (layer B.Cu) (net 35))
 (segment (start 42.8625 124.1425) (end 37.465 118.745) (width 0.25) (layer B.Cu) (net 35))
 (segment (start 109.538 129.988) (end 128.588 129.988) (width 0.25) (layer B.Cu) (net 19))
 (segment (start 80.9625 129.988) (end 109.538 129.988) (width 0.25) (layer B.Cu) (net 19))
 (segment (start 128.588 129.988) (end 157.162 129.988) (width 0.25) (layer B.Cu) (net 19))
 (segment (start 80.9625 129.988) (end 75.8669 129.988) (width 0.25) (layer B.Cu) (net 19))
 (segment (start 75.8669 129.988) (end 66.2109 120.332) (width 0.25) (layer B.Cu) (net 19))
 (segment (start 66.2109 120.332) (end 55.245 120.332) (width 0.25) (layer B.Cu) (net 19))
 (segment (start 55.245 120.332) (end 46.355 111.442) (width 0.25) (layer B.Cu) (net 19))
 (segment (start 42.8625 129.988) (end 42.8625 129.1127) (width 0.25) (layer B.Cu) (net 19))
 (segment (start 42.8625 129.1127) (end 43.7378 128.2374) (width 0.25) (layer B.Cu) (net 19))
 (segment (start 43.7378 128.2374) (end 43.7378 114.0592) (width 0.25) (layer B.Cu) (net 19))
 (segment (start 43.7378 114.0592) (end 46.355 111.442) (width 0.25) (layer B.Cu) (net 19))
 (segment (start 80.9625 127.188) (end 80.9625 124.1425) (width 0.25) (layer B.Cu) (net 34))
 (segment (start 80.9625 124.1425) (end 75.565 118.745) (width 0.25) (layer B.Cu) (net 34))
 (segment (start 109.538 127.188) (end 109.538 124.143) (width 0.25) (layer B.Cu) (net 33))
 (segment (start 109.538 124.143) (end 104.14 118.745) (width 0.25) (layer B.Cu) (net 33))
 (segment (start 128.588 127.188) (end 128.588 124.143) (width 0.25) (layer B.Cu) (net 32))
 (segment (start 128.588 124.143) (end 123.19 118.745) (width 0.25) (layer B.Cu) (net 32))
 (segment (start 157.162 127.188) (end 157.162 124.142) (width 0.25) (layer B.Cu) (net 31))
 (segment (start 157.162 124.142) (end 151.765 118.745) (width 0.25) (layer B.Cu) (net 31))
 (segment (start 42.8625 146.238) (end 42.8625 143.1925) (width 0.25) (layer B.Cu) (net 30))
 (segment (start 42.8625 143.1925) (end 37.465 137.795) (width 0.25) (layer B.Cu) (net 30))
 (segment (start 109.538 149.038) (end 157.162 149.038) (width 0.25) (layer B.Cu) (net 18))
 (segment (start 80.9625 149.038) (end 109.538 149.038) (width 0.25) (layer B.Cu) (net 18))
 (segment (start 61.9125 149.038) (end 80.9625 149.038) (width 0.25) (layer B.Cu) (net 18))
 (segment (start 45.1445 149.038) (end 61.9125 149.038) (width 0.25) (layer B.Cu) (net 18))
 (segment (start 42.8625 149.038) (end 45.1445 149.038) (width 0.25) (layer B.Cu) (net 18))
 (segment (start 45.1445 149.038) (end 45.1445 115.1925) (width 0.25) (layer B.Cu) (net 18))
 (segment (start 45.1445 115.1925) (end 46.355 113.982) (width 0.25) (layer B.Cu) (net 18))
 (segment (start 176.212 149.038) (end 157.162 149.038) (width 0.25) (layer B.Cu) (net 18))
 (segment (start 61.9125 146.238) (end 61.9125 143.1925) (width 0.25) (layer B.Cu) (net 29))
 (segment (start 61.9125 143.1925) (end 56.515 137.795) (width 0.25) (layer B.Cu) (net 29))
 (segment (start 80.9625 146.238) (end 80.9625 143.1925) (width 0.25) (layer B.Cu) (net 28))
 (segment (start 80.9625 143.1925) (end 75.565 137.795) (width 0.25) (layer B.Cu) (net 28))
 (segment (start 109.538 146.238) (end 109.538 143.193) (width 0.25) (layer B.Cu) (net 27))
 (segment (start 109.538 143.193) (end 104.14 137.795) (width 0.25) (layer B.Cu) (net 27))
 (segment (start 157.162 146.238) (end 157.162 143.192) (width 0.25) (layer B.Cu) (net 26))
 (segment (start 157.162 143.192) (end 151.765 137.795) (width 0.25) (layer B.Cu) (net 26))
 (segment (start 176.212 146.238) (end 176.212 143.192) (width 0.25) (layer B.Cu) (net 25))
 (segment (start 176.212 143.192) (end 170.815 137.795) (width 0.25) (layer B.Cu) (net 25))
 (segment (start 46.355 98.742) (end 45.1534 98.742) (width 0.25) (layer F.Cu) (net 24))
 (segment (start 31.115 102.235) (end 41.6604 102.235) (width 0.25) (layer F.Cu) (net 24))
 (segment (start 41.6604 102.235) (end 45.1534 98.742) (width 0.25) (layer F.Cu) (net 24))
 (segment (start 31.115 121.285) (end 31.115 140.335) (width 0.25) (layer B.Cu) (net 24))
 (segment (start 31.115 102.235) (end 31.115 121.285) (width 0.25) (layer B.Cu) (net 24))
 (segment (start 61.595 108.902) (end 60.3609 110.1361) (width 0.25) (layer F.Cu) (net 6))
 (segment (start 60.3609 110.1361) (end 60.3609 119.6001) (width 0.25) (layer F.Cu) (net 6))
 (segment (start 60.3609 119.6001) (end 61.0297 120.2689) (width 0.25) (layer F.Cu) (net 6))
 (segment (start 61.0297 120.2689) (end 68.1989 120.2689) (width 0.25) (layer F.Cu) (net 6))
 (segment (start 68.1989 120.2689) (end 69.215 121.285) (width 0.25) (layer F.Cu) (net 6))
 (segment (start 69.215 121.285) (end 69.215 140.335) (width 0.25) (layer F.Cu) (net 6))
 (segment (start 69.215 102.235) (end 68.262 102.235) (width 0.25) (layer B.Cu) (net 6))
 (segment (start 68.262 102.235) (end 61.595 108.902) (width 0.25) (layer B.Cu) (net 6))
 (segment (start 91.1188 111.6306) (end 61.7836 111.6306) (width 0.25) (layer B.Cu) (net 7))
 (segment (start 61.7836 111.6306) (end 61.595 111.442) (width 0.25) (layer B.Cu) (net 7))
 (segment (start 97.79 121.285) (end 97.79 118.3018) (width 0.25) (layer B.Cu) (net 7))
 (segment (start 97.79 118.3018) (end 91.1188 111.6306) (width 0.25) (layer B.Cu) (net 7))
 (segment (start 97.79 102.235) (end 97.337 102.235) (width 0.25) (layer B.Cu) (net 7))
 (segment (start 97.337 102.235) (end 91.1188 108.4532) (width 0.25) (layer B.Cu) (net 7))
 (segment (start 91.1188 108.4532) (end 91.1188 111.6306) (width 0.25) (layer B.Cu) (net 7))
 (segment (start 97.79 121.285) (end 97.79 140.335) (width 0.25) (layer F.Cu) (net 7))
 (segment (start 109.537 113.982) (end 61.595 113.982) (width 0.25) (layer F.Cu) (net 8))
 (segment (start 116.84 121.285) (end 109.537 113.982) (width 0.25) (layer F.Cu) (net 8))
 (segment (start 116.84 102.235) (end 116.84 106.679) (width 0.25) (layer F.Cu) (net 8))
 (segment (start 116.84 106.679) (end 109.537 113.982) (width 0.25) (layer F.Cu) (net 8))
 (segment (start 142.8962 123.272) (end 142.8962 137.8162) (width 0.25) (layer F.Cu) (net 9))
 (segment (start 142.8962 137.8162) (end 145.415 140.335) (width 0.25) (layer F.Cu) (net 9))
 (segment (start 145.415 121.285) (end 144.8832 121.285) (width 0.25) (layer F.Cu) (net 9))
 (segment (start 144.8832 121.285) (end 142.8962 123.272) (width 0.25) (layer F.Cu) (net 9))
 (segment (start 142.8962 123.272) (end 141.1203 121.4961) (width 0.25) (layer F.Cu) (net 9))
 (segment (start 141.1203 121.4961) (end 119.247 121.4961) (width 0.25) (layer F.Cu) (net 9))
 (segment (start 119.247 121.4961) (end 117.9782 122.7649) (width 0.25) (layer F.Cu) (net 9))
 (segment (start 117.9782 122.7649) (end 116.2688 122.7649) (width 0.25) (layer F.Cu) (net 9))
 (segment (start 116.2688 122.7649) (end 110.0259 116.522) (width 0.25) (layer F.Cu) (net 9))
 (segment (start 110.0259 116.522) (end 61.595 116.522) (width 0.25) (layer F.Cu) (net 9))
 (segment (start 145.415 102.235) (end 145.415 121.285) (width 0.25) (layer F.Cu) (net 9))
 (segment (start 50.165 140.335) (end 50.165 105.092) (width 0.25) (layer F.Cu) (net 23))
 (segment (start 50.165 105.092) (end 46.355 101.282) (width 0.25) (layer F.Cu) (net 23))
 (segment (start 164.465 140.335) (end 148.0331 140.335) (width 0.25) (layer F.Cu) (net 10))
 (segment (start 148.0331 140.335) (end 146.5532 141.8149) (width 0.25) (layer F.Cu) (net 10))
 (segment (start 146.5532 141.8149) (end 144.8438 141.8149) (width 0.25) (layer F.Cu) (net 10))
 (segment (start 144.8438 141.8149) (end 134.2953 131.2664) (width 0.25) (layer F.Cu) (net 10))
 (segment (start 134.2953 131.2664) (end 117.1726 131.2664) (width 0.25) (layer F.Cu) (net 10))
 (segment (start 117.1726 131.2664) (end 107.4119 121.5057) (width 0.25) (layer F.Cu) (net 10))
 (segment (start 107.4119 121.5057) (end 104.3608 121.5057) (width 0.25) (layer F.Cu) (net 10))
 (segment (start 104.3608 121.5057) (end 100.1104 117.2553) (width 0.25) (layer F.Cu) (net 10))
 (segment (start 100.1104 117.2553) (end 63.4017 117.2553) (width 0.25) (layer F.Cu) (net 10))
 (segment (start 63.4017 117.2553) (end 61.595 119.062) (width 0.25) (layer F.Cu) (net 10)))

